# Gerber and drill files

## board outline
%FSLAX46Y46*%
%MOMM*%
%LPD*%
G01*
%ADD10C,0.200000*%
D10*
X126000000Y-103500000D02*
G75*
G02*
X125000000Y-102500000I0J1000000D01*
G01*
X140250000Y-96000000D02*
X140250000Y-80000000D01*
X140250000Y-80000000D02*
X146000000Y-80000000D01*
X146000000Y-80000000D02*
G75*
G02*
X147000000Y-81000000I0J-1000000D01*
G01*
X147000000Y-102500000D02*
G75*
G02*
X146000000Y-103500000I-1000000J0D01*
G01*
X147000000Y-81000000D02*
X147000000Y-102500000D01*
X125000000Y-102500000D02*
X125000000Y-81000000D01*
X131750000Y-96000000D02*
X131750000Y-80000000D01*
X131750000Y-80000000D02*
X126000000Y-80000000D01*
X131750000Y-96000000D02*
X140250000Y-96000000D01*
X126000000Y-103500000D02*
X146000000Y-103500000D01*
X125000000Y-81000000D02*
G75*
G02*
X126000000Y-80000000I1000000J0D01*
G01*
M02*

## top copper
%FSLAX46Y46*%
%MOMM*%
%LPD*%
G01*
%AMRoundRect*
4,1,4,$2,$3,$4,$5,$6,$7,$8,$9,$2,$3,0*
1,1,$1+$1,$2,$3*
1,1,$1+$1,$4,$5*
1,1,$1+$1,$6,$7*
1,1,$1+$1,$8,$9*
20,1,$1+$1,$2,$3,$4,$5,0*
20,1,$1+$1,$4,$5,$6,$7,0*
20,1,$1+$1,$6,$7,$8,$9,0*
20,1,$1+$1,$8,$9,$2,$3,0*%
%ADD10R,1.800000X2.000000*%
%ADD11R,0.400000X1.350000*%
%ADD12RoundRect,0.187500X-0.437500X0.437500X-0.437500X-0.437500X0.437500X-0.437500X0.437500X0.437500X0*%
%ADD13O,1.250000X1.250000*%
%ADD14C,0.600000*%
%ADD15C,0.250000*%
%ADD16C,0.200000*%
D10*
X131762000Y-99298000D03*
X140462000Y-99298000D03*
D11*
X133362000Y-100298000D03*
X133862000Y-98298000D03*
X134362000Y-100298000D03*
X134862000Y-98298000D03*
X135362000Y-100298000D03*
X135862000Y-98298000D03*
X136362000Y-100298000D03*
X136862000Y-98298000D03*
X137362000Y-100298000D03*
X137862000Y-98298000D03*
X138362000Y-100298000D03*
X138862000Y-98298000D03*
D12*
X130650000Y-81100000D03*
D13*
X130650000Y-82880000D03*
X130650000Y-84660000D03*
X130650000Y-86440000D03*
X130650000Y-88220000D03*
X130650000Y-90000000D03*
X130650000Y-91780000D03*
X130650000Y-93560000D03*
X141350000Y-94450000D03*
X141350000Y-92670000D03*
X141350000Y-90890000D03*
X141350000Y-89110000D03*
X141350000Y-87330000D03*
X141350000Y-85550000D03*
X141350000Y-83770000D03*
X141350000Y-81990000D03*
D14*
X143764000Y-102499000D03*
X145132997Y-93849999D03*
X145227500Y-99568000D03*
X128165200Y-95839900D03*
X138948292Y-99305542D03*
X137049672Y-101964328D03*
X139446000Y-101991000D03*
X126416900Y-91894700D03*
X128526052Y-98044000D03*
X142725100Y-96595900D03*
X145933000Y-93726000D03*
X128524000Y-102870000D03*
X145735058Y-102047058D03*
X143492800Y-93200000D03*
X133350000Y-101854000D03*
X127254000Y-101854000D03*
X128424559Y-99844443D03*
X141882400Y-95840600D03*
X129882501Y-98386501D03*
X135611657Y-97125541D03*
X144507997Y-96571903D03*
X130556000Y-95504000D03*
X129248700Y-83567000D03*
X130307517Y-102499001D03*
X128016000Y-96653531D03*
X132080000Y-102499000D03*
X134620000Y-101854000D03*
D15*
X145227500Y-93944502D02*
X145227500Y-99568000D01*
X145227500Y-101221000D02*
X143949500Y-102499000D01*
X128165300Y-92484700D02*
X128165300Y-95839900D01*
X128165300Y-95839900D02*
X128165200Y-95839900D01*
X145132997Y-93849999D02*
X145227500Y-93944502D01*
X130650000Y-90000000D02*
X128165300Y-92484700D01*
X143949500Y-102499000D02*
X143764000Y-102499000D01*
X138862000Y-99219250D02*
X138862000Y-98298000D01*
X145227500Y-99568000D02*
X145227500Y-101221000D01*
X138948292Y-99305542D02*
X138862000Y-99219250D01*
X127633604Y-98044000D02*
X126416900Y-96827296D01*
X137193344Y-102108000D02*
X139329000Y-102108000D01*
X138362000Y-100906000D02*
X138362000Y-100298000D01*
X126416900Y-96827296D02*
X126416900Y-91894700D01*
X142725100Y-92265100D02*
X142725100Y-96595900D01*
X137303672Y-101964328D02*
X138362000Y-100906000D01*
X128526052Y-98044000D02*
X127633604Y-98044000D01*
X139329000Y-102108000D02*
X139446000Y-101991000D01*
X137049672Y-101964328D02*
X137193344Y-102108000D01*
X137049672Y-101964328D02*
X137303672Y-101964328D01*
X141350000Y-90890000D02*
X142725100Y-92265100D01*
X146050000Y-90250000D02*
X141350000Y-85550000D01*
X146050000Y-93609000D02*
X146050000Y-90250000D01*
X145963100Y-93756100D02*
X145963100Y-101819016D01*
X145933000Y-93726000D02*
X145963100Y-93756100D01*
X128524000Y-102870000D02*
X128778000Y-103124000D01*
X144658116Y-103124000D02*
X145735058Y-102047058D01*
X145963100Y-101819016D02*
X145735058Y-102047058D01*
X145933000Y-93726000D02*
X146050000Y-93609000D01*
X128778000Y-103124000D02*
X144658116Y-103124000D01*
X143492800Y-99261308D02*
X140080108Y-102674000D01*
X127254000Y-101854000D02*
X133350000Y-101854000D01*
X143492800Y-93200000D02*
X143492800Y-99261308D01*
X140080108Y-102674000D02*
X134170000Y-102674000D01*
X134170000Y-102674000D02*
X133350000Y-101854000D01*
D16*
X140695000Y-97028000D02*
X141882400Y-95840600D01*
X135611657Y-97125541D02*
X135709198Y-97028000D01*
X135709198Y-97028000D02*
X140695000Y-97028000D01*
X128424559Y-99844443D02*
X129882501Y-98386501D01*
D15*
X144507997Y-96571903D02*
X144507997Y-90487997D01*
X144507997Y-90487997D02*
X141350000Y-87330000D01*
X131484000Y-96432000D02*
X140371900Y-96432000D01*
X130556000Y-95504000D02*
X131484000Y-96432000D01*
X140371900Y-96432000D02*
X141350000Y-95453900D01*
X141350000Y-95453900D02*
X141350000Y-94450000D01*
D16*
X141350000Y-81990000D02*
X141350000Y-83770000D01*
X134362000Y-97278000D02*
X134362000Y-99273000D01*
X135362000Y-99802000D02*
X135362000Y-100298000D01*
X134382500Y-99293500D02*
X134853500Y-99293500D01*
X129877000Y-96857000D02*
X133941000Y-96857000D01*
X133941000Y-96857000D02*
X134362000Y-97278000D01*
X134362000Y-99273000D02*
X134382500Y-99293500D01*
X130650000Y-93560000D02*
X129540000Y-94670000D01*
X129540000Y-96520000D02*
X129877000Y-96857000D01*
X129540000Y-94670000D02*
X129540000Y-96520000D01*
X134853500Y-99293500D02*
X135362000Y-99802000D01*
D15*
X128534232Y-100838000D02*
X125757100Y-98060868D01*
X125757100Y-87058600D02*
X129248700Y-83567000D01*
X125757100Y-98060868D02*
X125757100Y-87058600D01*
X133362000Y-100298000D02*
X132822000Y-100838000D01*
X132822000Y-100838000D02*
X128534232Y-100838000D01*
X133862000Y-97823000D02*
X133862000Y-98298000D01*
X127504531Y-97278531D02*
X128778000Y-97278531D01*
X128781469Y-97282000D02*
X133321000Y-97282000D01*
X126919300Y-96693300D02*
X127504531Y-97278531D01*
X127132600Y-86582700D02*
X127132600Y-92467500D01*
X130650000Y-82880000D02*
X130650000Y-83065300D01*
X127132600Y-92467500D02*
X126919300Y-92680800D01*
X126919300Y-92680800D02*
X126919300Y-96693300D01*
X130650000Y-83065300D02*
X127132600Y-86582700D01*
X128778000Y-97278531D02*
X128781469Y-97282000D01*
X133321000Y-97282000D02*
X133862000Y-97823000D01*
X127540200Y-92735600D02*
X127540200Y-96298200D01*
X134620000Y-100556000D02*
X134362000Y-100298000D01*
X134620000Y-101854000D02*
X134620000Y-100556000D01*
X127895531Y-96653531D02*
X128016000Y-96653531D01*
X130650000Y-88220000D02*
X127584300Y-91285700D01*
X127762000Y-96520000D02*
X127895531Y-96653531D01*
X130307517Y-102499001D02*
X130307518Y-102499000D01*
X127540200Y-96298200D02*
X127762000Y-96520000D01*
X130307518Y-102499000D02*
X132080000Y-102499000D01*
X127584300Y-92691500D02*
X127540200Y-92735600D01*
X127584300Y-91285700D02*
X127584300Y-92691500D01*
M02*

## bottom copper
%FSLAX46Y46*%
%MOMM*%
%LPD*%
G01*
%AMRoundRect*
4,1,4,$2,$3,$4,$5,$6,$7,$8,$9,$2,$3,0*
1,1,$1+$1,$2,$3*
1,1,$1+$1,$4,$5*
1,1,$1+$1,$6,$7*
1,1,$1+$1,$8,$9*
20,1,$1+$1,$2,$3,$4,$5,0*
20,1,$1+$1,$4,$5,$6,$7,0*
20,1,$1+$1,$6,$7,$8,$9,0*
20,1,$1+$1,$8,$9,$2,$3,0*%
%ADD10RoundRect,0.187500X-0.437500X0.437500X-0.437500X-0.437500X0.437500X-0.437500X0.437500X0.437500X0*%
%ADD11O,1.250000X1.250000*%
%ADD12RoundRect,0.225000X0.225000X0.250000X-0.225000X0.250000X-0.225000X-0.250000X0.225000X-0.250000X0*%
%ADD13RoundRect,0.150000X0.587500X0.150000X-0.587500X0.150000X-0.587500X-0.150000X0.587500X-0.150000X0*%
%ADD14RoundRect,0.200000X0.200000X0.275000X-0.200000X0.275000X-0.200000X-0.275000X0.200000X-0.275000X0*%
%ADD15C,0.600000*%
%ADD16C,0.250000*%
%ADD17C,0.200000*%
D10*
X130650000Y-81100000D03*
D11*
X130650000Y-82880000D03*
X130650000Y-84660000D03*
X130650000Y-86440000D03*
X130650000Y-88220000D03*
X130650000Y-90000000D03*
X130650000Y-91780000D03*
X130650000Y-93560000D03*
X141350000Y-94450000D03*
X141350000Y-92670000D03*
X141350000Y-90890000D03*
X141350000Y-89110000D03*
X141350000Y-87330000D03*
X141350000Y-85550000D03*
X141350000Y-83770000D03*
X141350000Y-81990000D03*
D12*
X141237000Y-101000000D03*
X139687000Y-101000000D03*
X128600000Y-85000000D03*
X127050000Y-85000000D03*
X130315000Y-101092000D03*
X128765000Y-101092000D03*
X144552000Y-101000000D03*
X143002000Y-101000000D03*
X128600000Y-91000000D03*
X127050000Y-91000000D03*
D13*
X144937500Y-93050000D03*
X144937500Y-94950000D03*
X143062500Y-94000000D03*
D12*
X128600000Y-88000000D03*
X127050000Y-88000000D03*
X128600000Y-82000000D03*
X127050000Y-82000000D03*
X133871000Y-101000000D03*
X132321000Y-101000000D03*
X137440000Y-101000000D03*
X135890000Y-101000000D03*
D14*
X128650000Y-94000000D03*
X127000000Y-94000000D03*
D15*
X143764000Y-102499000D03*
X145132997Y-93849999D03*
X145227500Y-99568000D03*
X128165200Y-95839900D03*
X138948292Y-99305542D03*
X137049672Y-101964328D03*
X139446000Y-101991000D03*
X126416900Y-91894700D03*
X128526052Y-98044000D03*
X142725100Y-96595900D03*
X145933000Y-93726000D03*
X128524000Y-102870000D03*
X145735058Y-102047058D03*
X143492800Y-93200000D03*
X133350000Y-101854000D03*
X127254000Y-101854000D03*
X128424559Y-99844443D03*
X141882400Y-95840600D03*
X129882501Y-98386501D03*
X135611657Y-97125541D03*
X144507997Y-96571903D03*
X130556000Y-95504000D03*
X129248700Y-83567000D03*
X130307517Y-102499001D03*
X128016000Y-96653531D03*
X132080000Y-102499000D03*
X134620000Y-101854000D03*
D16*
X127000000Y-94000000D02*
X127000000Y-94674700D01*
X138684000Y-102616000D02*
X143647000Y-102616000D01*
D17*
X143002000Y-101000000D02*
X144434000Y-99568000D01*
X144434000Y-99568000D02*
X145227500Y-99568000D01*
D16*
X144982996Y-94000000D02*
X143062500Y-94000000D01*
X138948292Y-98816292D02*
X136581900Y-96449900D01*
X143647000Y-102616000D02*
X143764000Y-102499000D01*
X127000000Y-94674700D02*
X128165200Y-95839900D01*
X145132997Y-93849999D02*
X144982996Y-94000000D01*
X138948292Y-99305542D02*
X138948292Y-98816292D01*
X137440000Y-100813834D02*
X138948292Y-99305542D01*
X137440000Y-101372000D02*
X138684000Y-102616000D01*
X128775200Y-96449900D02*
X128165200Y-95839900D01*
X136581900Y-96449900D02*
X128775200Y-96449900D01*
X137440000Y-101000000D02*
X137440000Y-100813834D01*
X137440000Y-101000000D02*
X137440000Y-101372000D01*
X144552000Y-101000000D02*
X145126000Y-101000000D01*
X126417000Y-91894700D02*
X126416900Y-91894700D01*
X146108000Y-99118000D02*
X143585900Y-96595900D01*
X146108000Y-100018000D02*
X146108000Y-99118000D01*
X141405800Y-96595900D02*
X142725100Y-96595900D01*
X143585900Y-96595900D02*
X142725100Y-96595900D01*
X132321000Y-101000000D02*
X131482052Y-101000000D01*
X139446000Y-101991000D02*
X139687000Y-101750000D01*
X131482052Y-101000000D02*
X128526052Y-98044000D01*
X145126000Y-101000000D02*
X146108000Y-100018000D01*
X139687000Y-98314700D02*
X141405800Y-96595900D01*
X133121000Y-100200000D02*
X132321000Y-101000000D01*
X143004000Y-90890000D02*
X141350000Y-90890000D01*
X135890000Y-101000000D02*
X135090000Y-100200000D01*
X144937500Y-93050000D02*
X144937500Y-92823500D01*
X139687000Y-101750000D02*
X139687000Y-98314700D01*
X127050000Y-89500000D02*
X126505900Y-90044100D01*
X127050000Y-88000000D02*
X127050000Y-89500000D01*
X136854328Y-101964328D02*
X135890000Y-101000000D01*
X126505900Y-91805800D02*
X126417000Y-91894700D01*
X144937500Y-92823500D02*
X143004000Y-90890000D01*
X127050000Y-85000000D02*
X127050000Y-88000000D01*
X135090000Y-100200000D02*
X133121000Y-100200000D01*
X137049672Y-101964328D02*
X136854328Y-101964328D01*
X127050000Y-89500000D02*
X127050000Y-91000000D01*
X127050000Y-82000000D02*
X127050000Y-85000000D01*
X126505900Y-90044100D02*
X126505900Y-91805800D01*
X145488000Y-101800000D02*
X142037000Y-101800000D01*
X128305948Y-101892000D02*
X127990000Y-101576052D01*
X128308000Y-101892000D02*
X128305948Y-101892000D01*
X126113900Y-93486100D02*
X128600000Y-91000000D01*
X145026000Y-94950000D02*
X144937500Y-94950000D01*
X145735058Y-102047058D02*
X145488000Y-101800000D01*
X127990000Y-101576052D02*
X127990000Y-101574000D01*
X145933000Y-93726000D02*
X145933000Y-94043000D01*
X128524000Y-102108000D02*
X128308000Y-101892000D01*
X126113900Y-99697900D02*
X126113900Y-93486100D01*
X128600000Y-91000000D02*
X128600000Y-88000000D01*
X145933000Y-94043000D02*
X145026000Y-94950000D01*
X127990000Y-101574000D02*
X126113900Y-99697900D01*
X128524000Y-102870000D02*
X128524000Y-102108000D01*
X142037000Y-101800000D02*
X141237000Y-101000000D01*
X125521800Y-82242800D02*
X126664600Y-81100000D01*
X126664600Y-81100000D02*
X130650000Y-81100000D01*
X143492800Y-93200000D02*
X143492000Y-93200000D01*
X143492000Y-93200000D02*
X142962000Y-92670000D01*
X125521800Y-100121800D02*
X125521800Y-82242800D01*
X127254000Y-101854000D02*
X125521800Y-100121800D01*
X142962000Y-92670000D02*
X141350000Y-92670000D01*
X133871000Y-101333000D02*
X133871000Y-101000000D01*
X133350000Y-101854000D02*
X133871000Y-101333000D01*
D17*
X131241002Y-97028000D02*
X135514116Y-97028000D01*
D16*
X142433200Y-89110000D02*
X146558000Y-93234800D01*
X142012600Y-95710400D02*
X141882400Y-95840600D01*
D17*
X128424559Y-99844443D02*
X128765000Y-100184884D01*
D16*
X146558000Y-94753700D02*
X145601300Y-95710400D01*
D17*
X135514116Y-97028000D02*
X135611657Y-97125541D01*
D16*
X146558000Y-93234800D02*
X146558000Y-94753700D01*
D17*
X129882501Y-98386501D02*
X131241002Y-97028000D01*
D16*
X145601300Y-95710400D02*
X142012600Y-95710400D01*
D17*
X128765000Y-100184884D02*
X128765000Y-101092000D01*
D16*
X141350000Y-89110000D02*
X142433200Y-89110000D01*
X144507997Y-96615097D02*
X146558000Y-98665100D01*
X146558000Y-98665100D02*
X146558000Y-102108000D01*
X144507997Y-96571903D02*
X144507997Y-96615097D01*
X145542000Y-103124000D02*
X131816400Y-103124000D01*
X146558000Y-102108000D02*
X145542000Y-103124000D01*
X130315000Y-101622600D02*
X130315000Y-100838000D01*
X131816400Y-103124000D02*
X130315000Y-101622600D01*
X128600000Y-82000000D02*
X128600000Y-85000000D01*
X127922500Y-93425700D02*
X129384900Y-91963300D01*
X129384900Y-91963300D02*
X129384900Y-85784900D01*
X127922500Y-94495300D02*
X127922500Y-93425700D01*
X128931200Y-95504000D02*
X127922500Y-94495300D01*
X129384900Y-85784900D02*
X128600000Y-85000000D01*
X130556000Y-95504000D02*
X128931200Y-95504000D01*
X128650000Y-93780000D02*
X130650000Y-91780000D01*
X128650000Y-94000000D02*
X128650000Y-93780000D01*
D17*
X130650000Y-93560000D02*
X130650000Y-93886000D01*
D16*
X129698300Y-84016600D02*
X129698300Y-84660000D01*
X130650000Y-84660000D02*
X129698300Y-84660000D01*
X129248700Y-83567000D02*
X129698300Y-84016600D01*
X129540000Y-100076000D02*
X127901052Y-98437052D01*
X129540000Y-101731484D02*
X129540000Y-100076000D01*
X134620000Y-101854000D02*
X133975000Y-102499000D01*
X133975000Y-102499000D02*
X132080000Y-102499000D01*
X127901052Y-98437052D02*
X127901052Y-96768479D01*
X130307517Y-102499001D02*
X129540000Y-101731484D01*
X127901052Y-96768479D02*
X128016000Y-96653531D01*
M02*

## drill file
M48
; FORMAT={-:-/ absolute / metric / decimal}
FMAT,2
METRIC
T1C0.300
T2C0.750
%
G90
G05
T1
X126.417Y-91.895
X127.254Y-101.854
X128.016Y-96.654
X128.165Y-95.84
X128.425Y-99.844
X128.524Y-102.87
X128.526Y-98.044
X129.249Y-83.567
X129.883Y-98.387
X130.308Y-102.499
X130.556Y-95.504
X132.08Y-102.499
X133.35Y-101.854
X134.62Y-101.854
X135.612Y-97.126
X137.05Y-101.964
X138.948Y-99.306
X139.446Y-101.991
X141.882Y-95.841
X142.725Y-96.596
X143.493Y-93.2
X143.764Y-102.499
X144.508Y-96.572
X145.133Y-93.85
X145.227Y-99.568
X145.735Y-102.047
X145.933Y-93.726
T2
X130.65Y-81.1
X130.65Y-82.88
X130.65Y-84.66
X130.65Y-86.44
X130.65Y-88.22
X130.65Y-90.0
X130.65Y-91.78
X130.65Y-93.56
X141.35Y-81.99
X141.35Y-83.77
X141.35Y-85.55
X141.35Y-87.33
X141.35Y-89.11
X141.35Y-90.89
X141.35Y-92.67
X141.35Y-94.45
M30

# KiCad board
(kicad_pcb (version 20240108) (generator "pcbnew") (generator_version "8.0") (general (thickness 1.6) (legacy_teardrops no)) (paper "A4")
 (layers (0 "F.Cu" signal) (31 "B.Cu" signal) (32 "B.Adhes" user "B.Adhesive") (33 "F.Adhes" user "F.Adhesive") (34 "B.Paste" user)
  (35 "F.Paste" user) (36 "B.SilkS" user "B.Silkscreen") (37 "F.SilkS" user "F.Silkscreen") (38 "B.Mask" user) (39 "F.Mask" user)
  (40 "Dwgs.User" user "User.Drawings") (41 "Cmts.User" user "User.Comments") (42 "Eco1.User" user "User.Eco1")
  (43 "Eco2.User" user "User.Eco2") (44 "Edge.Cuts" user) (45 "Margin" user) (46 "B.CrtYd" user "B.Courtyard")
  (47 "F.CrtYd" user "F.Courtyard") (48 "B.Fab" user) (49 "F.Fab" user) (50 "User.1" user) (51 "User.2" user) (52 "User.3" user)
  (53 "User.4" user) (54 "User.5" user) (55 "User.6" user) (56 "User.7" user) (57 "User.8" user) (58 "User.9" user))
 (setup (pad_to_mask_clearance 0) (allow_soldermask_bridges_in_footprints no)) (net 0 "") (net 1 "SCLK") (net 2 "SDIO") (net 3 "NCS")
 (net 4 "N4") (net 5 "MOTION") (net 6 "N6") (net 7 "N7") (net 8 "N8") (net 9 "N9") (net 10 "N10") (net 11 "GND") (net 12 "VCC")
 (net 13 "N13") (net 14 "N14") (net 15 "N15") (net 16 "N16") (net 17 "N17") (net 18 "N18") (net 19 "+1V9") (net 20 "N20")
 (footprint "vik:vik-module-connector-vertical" (layer "F.Cu") (at 136.112 99.298)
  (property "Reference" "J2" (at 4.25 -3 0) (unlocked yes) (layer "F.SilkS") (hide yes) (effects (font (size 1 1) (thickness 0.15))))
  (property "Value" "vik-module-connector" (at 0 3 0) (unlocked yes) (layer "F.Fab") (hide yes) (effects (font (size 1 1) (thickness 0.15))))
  (pad "" smd rect (at -4.35 0) (size 1.8 2) (layers "F.Cu" "F.Paste" "F.Mask") (thermal_bridge_angle 45))
  (pad "" smd rect (at 4.35 0) (size 1.8 2) (layers "F.Cu" "F.Paste" "F.Mask") (thermal_bridge_angle 45))
  (pad "1" smd rect (at -2.75 1) (size 0.4 1.35) (layers "F.Cu" "F.Paste" "F.Mask") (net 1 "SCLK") (thermal_bridge_angle 45))
  (pad "2" smd rect (at -2.25 -1) (size 0.4 1.35) (layers "F.Cu" "F.Paste" "F.Mask") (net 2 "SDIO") (thermal_bridge_angle 45))
  (pad "3" smd rect (at -1.75 1) (size 0.4 1.35) (layers "F.Cu" "F.Paste" "F.Mask") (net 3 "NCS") (thermal_bridge_angle 45))
  (pad "4" smd rect (at -1.25 -1) (size 0.4 1.35) (layers "F.Cu" "F.Paste" "F.Mask") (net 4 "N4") (thermal_bridge_angle 45))
  (pad "5" smd rect (at -0.75 1) (size 0.4 1.35) (layers "F.Cu" "F.Paste" "F.Mask") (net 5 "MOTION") (thermal_bridge_angle 45))
  (pad "6" smd rect (at -0.25 -1) (size 0.4 1.35) (layers "F.Cu" "F.Paste" "F.Mask") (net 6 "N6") (thermal_bridge_angle 45))
  (pad "7" smd rect (at 0.25 1) (size 0.4 1.35) (layers "F.Cu" "F.Paste" "F.Mask") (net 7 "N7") (thermal_bridge_angle 45))
  (pad "8" smd rect (at 0.75 -1) (size 0.4 1.35) (layers "F.Cu" "F.Paste" "F.Mask") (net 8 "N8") (thermal_bridge_angle 45))
  (pad "9" smd rect (at 1.25 1) (size 0.4 1.35) (layers "F.Cu" "F.Paste" "F.Mask") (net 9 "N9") (thermal_bridge_angle 45))
  (pad "10" smd rect (at 1.75 -1) (size 0.4 1.35) (layers "F.Cu" "F.Paste" "F.Mask") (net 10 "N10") (thermal_bridge_angle 45))
  (pad "11" smd rect (at 2.25 1) (size 0.4 1.35) (layers "F.Cu" "F.Paste" "F.Mask") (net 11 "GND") (thermal_bridge_angle 45))
  (pad "12" smd rect (at 2.75 -1) (size 0.4 1.35) (layers "F.Cu" "F.Paste" "F.Mask") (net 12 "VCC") (thermal_bridge_angle 45)))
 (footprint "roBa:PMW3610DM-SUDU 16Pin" (layer "F.Cu") (at 136 87.268 90)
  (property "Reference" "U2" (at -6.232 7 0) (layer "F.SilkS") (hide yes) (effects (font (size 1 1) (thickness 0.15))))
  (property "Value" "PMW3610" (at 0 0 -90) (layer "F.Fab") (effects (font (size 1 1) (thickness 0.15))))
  (pad "1" thru_hole roundrect (at 6.168 -5.35 270) (size 1.25 1.25) (drill 0.75) (layers "*.Cu" "*.Mask") (remove_unused_layers no)
   (roundrect_rratio 0.15) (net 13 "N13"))
  (pad "2" thru_hole oval (at 4.388 -5.35 270) (size 1.25 1.25) (drill 0.75) (layers "*.Cu" "*.Mask") (remove_unused_layers no)
   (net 2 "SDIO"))
  (pad "3" thru_hole oval (at 2.608 -5.35 270) (size 1.25 1.25) (drill 0.75) (layers "*.Cu" "*.Mask") (remove_unused_layers no)
   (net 1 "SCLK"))
  (pad "4" thru_hole oval (at 0.828 -5.35 270) (size 1.25 1.25) (drill 0.75) (layers "*.Cu" "*.Mask") (remove_unused_layers no)
   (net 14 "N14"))
  (pad "5" thru_hole oval (at -0.952 -5.35 270) (size 1.25 1.25) (drill 0.75) (layers "*.Cu" "*.Mask") (remove_unused_layers no)
   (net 3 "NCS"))
  (pad "6" thru_hole oval (at -2.732 -5.35 270) (size 1.25 1.25) (drill 0.75) (layers "*.Cu" "*.Mask") (remove_unused_layers no)
   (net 12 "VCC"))
  (pad "7" thru_hole oval (at -4.512 -5.35 270) (size 1.25 1.25) (drill 0.75) (layers "*.Cu" "*.Mask") (remove_unused_layers no)
   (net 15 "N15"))
  (pad "8" thru_hole oval (at -6.292 -5.35 270) (size 1.25 1.25) (drill 0.75) (layers "*.Cu" "*.Mask") (remove_unused_layers no)
   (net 5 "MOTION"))
  (pad "9" thru_hole oval (at -7.182 5.35 270) (size 1.25 1.25) (drill 0.75) (layers "*.Cu" "*.Mask") (remove_unused_layers no)
   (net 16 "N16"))
  (pad "10" thru_hole oval (at -5.402 5.35 270) (size 1.25 1.25) (drill 0.75) (layers "*.Cu" "*.Mask") (remove_unused_layers no)
   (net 13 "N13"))
  (pad "11" thru_hole oval (at -3.622 5.35 270) (size 1.25 1.25) (drill 0.75) (layers "*.Cu" "*.Mask") (remove_unused_layers no)
   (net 11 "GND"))
  (pad "12" thru_hole oval (at -1.842 5.35 270) (size 1.25 1.25) (drill 0.75) (layers "*.Cu" "*.Mask") (remove_unused_layers no)
   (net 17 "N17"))
  (pad "13" thru_hole oval (at -0.062 5.35 270) (size 1.25 1.25) (drill 0.75) (layers "*.Cu" "*.Mask") (remove_unused_layers no)
   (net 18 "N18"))
  (pad "14" thru_hole oval (at 1.718 5.35 270) (size 1.25 1.25) (drill 0.75) (layers "*.Cu" "*.Mask") (remove_unused_layers no)
   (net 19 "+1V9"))
  (pad "15" thru_hole oval (at 3.498 5.35 270) (size 1.25 1.25) (drill 0.75) (layers "*.Cu" "*.Mask") (remove_unused_layers no)
   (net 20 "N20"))
  (pad "16" thru_hole oval (at 5.278 5.35 270) (size 1.25 1.25) (drill 0.75) (layers "*.Cu" "*.Mask") (remove_unused_layers no)
   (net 20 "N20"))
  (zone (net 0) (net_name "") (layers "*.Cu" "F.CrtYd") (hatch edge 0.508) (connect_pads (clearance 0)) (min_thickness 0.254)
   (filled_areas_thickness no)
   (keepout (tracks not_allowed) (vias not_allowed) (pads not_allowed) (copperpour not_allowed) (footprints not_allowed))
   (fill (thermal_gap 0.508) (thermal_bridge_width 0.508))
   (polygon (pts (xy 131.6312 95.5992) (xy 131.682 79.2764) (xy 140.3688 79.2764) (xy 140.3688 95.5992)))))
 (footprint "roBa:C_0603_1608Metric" (layer "B.Cu") (at 140.462 101 180)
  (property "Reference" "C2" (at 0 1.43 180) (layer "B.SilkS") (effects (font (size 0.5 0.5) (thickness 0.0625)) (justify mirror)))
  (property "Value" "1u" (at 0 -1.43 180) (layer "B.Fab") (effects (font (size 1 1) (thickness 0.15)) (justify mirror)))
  (pad "1" smd roundrect (at -0.775 0 180) (size 0.9 0.95) (layers "B.Cu" "B.Paste" "B.Mask") (roundrect_rratio 0.25) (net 19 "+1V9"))
  (pad "2" smd roundrect (at 0.775 0 180) (size 0.9 0.95) (layers "B.Cu" "B.Paste" "B.Mask") (roundrect_rratio 0.25) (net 11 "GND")))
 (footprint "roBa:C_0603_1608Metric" (layer "B.Cu") (at 127.825 85 180)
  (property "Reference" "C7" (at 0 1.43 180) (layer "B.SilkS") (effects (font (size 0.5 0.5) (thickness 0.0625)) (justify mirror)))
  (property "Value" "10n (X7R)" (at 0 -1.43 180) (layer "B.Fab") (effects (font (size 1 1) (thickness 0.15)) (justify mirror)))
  (pad "1" smd roundrect (at -0.775 0 180) (size 0.9 0.95) (layers "B.Cu" "B.Paste" "B.Mask") (roundrect_rratio 0.25) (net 16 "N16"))
  (pad "2" smd roundrect (at 0.775 0 180) (size 0.9 0.95) (layers "B.Cu" "B.Paste" "B.Mask") (roundrect_rratio 0.25) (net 11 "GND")))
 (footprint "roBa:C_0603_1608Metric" (layer "B.Cu") (at 129.54 101.092 180)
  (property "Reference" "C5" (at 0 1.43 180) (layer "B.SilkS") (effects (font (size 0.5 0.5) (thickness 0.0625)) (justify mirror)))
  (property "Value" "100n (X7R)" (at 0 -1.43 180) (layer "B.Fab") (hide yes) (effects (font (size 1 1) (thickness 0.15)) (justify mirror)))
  (pad "1" smd roundrect (at -0.775 0 180) (size 0.9 0.95) (layers "B.Cu" "B.Paste" "B.Mask") (roundrect_rratio 0.25) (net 18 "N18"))
  (pad "2" smd roundrect (at 0.775 0 180) (size 0.9 0.95) (layers "B.Cu" "B.Paste" "B.Mask") (roundrect_rratio 0.25) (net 17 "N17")))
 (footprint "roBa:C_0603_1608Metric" (layer "B.Cu") (at 143.777 101 180)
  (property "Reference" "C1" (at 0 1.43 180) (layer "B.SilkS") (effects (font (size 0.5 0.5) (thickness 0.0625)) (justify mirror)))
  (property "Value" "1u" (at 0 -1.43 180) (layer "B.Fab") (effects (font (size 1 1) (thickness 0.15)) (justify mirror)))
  (pad "1" smd roundrect (at -0.775 0 180) (size 0.9 0.95) (layers "B.Cu" "B.Paste" "B.Mask") (roundrect_rratio 0.25) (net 11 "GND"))
  (pad "2" smd roundrect (at 0.775 0 180) (size 0.9 0.95) (layers "B.Cu" "B.Paste" "B.Mask") (roundrect_rratio 0.25) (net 12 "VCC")))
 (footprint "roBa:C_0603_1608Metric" (layer "B.Cu") (at 127.825 91 180)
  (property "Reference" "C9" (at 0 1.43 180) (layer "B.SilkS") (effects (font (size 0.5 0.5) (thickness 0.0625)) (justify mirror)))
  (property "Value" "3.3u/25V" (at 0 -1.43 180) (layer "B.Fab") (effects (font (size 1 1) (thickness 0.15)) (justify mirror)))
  (pad "1" smd roundrect (at -0.775 0 180) (size 0.9 0.95) (layers "B.Cu" "B.Paste" "B.Mask") (roundrect_rratio 0.25) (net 19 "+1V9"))
  (pad "2" smd roundrect (at 0.775 0 180) (size 0.9 0.95) (layers "B.Cu" "B.Paste" "B.Mask") (roundrect_rratio 0.25) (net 11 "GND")))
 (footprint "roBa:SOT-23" (layer "B.Cu") (at 144 94 180)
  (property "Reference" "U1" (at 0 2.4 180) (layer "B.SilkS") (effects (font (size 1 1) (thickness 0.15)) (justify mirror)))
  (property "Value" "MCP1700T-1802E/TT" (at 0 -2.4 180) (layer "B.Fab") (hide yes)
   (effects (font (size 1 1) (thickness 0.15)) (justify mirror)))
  (pad "1" smd roundrect (at -0.9375 0.95 180) (size 1.475 0.6) (layers "B.Cu" "B.Paste" "B.Mask") (roundrect_rratio 0.25) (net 11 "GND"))
  (pad "2" smd roundrect (at -0.9375 -0.95 180) (size 1.475 0.6) (layers "B.Cu" "B.Paste" "B.Mask") (roundrect_rratio 0.25) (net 19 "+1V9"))
  (pad "3" smd roundrect (at 0.9375 0 180) (size 1.475 0.6) (layers "B.Cu" "B.Paste" "B.Mask") (roundrect_rratio 0.25) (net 12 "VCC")))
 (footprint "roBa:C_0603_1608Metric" (layer "B.Cu") (at 127.825 88 180)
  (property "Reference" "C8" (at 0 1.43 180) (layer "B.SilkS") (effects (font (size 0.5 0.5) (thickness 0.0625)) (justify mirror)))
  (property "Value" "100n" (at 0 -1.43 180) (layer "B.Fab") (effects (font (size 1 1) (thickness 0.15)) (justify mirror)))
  (pad "1" smd roundrect (at -0.775 0 180) (size 0.9 0.95) (layers "B.Cu" "B.Paste" "B.Mask") (roundrect_rratio 0.25) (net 19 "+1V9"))
  (pad "2" smd roundrect (at 0.775 0 180) (size 0.9 0.95) (layers "B.Cu" "B.Paste" "B.Mask") (roundrect_rratio 0.25) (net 11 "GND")))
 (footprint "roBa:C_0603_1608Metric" (layer "B.Cu") (at 127.825 82 180)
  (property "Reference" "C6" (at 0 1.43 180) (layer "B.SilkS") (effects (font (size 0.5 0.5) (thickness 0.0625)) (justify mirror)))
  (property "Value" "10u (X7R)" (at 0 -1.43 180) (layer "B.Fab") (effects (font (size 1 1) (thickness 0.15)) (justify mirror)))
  (pad "1" smd roundrect (at -0.775 0 180) (size 0.9 0.95) (layers "B.Cu" "B.Paste" "B.Mask") (roundrect_rratio 0.25) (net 16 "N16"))
  (pad "2" smd roundrect (at 0.775 0 180) (size 0.9 0.95) (layers "B.Cu" "B.Paste" "B.Mask") (roundrect_rratio 0.25) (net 11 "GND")))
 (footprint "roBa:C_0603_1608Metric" (layer "B.Cu") (at 133.096 101 180)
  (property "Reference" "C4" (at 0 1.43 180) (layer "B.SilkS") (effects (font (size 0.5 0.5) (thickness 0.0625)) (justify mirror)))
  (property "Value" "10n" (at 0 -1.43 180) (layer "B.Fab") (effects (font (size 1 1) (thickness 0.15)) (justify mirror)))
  (pad "1" smd roundrect (at -0.775 0 180) (size 0.9 0.95) (layers "B.Cu" "B.Paste" "B.Mask") (roundrect_rratio 0.25) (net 13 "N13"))
  (pad "2" smd roundrect (at 0.775 0 180) (size 0.9 0.95) (layers "B.Cu" "B.Paste" "B.Mask") (roundrect_rratio 0.25) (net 11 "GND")))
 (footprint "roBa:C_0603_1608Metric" (layer "B.Cu") (at 136.665 101 180)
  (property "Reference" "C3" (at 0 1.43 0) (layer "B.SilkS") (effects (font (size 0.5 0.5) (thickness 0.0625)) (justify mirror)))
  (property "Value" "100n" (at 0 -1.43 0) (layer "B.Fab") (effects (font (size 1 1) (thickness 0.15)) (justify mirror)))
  (pad "1" smd roundrect (at -0.775 0 180) (size 0.9 0.95) (layers "B.Cu" "B.Paste" "B.Mask") (roundrect_rratio 0.25) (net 12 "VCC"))
  (pad "2" smd roundrect (at 0.775 0 180) (size 0.9 0.95) (layers "B.Cu" "B.Paste" "B.Mask") (roundrect_rratio 0.25) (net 11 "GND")))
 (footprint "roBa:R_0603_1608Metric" (layer "B.Cu") (at 127.825 94 180)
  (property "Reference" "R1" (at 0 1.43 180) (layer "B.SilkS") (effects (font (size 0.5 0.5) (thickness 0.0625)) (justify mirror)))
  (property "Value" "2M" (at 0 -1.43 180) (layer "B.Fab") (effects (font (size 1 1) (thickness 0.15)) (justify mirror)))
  (pad "1" smd roundrect (at -0.825 0 180) (size 0.8 0.95) (layers "B.Cu" "B.Paste" "B.Mask") (roundrect_rratio 0.25) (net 15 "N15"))
  (pad "2" smd roundrect (at 0.825 0 180) (size 0.8 0.95) (layers "B.Cu" "B.Paste" "B.Mask") (roundrect_rratio 0.25) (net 12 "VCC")))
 (gr_arc (start 126 103.5) (mid 125.292893 103.207107) (end 125 102.5) (stroke (width 0.2) (type default)) (layer "Edge.Cuts"))
 (gr_line (start 140.25 96) (end 140.25 80) (stroke (width 0.2) (type default)) (layer "Edge.Cuts"))
 (gr_line (start 140.25 80) (end 146 80) (stroke (width 0.2) (type default)) (layer "Edge.Cuts"))
 (gr_arc (start 146 80) (mid 146.707107 80.292893) (end 147 81) (stroke (width 0.2) (type default)) (layer "Edge.Cuts"))
 (gr_arc (start 147 102.5) (mid 146.707107 103.207107) (end 146 103.5) (stroke (width 0.2) (type default)) (layer "Edge.Cuts"))
 (gr_line (start 147 81) (end 147 102.5) (stroke (width 0.2) (type default)) (layer "Edge.Cuts"))
 (gr_line (start 125 102.5) (end 125 81) (stroke (width 0.2) (type default)) (layer "Edge.Cuts"))
 (gr_line (start 131.75 96) (end 131.75 80) (stroke (width 0.2) (type default)) (layer "Edge.Cuts"))
 (gr_line (start 131.75 80) (end 126 80) (stroke (width 0.2) (type default)) (layer "Edge.Cuts"))
 (gr_line (start 131.75 96) (end 140.25 96) (stroke (width 0.2) (type default)) (layer "Edge.Cuts"))
 (gr_line (start 126 103.5) (end 146 103.5) (stroke (width 0.2) (type default)) (layer "Edge.Cuts"))
 (gr_arc (start 125 81) (mid 125.292893 80.292893) (end 126 80) (stroke (width 0.2) (type default)) (layer "Edge.Cuts"))
 (segment (start 145.2275 93.944502) (end 145.2275 99.568) (width 0.25) (layer "F.Cu") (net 12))
 (segment (start 145.2275 101.221) (end 143.9495 102.499) (width 0.25) (layer "F.Cu") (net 12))
 (segment (start 128.1653 92.4847) (end 128.1653 95.8399) (width 0.25) (layer "F.Cu") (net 12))
 (segment (start 128.1653 95.8399) (end 128.1652 95.8399) (width 0.25) (layer "F.Cu") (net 12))
 (segment (start 145.132997 93.849999) (end 145.2275 93.944502) (width 0.25) (layer "F.Cu") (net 12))
 (segment (start 130.65 90) (end 128.1653 92.4847) (width 0.25) (layer "F.Cu") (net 12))
 (segment (start 143.9495 102.499) (end 143.764 102.499) (width 0.25) (layer "F.Cu") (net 12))
 (segment (start 138.862 99.21925) (end 138.862 98.298) (width 0.25) (layer "F.Cu") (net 12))
 (segment (start 145.2275 99.568) (end 145.2275 101.221) (width 0.25) (layer "F.Cu") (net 12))
 (segment (start 138.948292 99.305542) (end 138.862 99.21925) (width 0.25) (layer "F.Cu") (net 12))
 (via (at 143.764 102.499) (size 0.6) (drill 0.3) (layers "F.Cu" "B.Cu") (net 12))
 (via (at 145.132997 93.849999) (size 0.6) (drill 0.3) (layers "F.Cu" "B.Cu") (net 12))
 (via (at 145.2275 99.568) (size 0.6) (drill 0.3) (layers "F.Cu" "B.Cu") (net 12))
 (via (at 128.1652 95.8399) (size 0.6) (drill 0.3) (layers "F.Cu" "B.Cu") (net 12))
 (via (at 138.948292 99.305542) (size 0.6) (drill 0.3) (layers "F.Cu" "B.Cu") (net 12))
 (segment (start 127 94) (end 127 94.6747) (width 0.25) (layer "B.Cu") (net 12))
 (segment (start 138.684 102.616) (end 143.647 102.616) (width 0.25) (layer "B.Cu") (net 12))
 (segment (start 143.002 101) (end 144.434 99.568) (width 0.2) (layer "B.Cu") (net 12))
 (segment (start 144.434 99.568) (end 145.2275 99.568) (width 0.2) (layer "B.Cu") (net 12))
 (segment (start 144.982996 94) (end 143.0625 94) (width 0.25) (layer "B.Cu") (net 12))
 (segment (start 138.948292 98.816292) (end 136.5819 96.4499) (width 0.25) (layer "B.Cu") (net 12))
 (segment (start 143.647 102.616) (end 143.764 102.499) (width 0.25) (layer "B.Cu") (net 12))
 (segment (start 127 94.6747) (end 128.1652 95.8399) (width 0.25) (layer "B.Cu") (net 12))
 (segment (start 145.132997 93.849999) (end 144.982996 94) (width 0.25) (layer "B.Cu") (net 12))
 (segment (start 138.948292 99.305542) (end 138.948292 98.816292) (width 0.25) (layer "B.Cu") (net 12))
 (segment (start 137.44 100.813834) (end 138.948292 99.305542) (width 0.25) (layer "B.Cu") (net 12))
 (segment (start 137.44 101.372) (end 138.684 102.616) (width 0.25) (layer "B.Cu") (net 12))
 (segment (start 128.7752 96.4499) (end 128.1652 95.8399) (width 0.25) (layer "B.Cu") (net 12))
 (segment (start 136.5819 96.4499) (end 128.7752 96.4499) (width 0.25) (layer "B.Cu") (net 12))
 (segment (start 137.44 101) (end 137.44 100.813834) (width 0.25) (layer "B.Cu") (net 12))
 (segment (start 137.44 101) (end 137.44 101.372) (width 0.25) (layer "B.Cu") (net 12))
 (segment (start 127.633604 98.044) (end 126.4169 96.827296) (width 0.25) (layer "F.Cu") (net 11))
 (segment (start 137.193344 102.108) (end 139.329 102.108) (width 0.25) (layer "F.Cu") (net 11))
 (segment (start 138.362 100.906) (end 138.362 100.298) (width 0.25) (layer "F.Cu") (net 11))
 (segment (start 126.4169 96.827296) (end 126.4169 91.8947) (width 0.25) (layer "F.Cu") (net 11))
 (segment (start 142.7251 92.2651) (end 142.7251 96.5959) (width 0.25) (layer "F.Cu") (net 11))
 (segment (start 137.303672 101.964328) (end 138.362 100.906) (width 0.25) (layer "F.Cu") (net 11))
 (segment (start 128.526052 98.044) (end 127.633604 98.044) (width 0.25) (layer "F.Cu") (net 11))
 (segment (start 139.329 102.108) (end 139.446 101.991) (width 0.25) (layer "F.Cu") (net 11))
 (segment (start 137.049672 101.964328) (end 137.193344 102.108) (width 0.25) (layer "F.Cu") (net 11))
 (segment (start 137.049672 101.964328) (end 137.303672 101.964328) (width 0.25) (layer "F.Cu") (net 11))
 (segment (start 141.35 90.89) (end 142.7251 92.2651) (width 0.25) (layer "F.Cu") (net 11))
 (via (at 137.049672 101.964328) (size 0.6) (drill 0.3) (layers "F.Cu" "B.Cu") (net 11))
 (via (at 139.446 101.991) (size 0.6) (drill 0.3) (layers "F.Cu" "B.Cu") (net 11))
 (via (at 126.4169 91.8947) (size 0.6) (drill 0.3) (layers "F.Cu" "B.Cu") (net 11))
 (via (at 128.526052 98.044) (size 0.6) (drill 0.3) (layers "F.Cu" "B.Cu") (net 11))
 (via (at 142.7251 96.5959) (size 0.6) (drill 0.3) (layers "F.Cu" "B.Cu") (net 11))
 (segment (start 144.552 101) (end 145.126 101) (width 0.25) (layer "B.Cu") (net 11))
 (segment (start 126.417 91.8947) (end 126.4169 91.8947) (width 0.25) (layer "B.Cu") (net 11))
 (segment (start 146.108 99.118) (end 143.5859 96.5959) (width 0.25) (layer "B.Cu") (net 11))
 (segment (start 146.108 100.018) (end 146.108 99.118) (width 0.25) (layer "B.Cu") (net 11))
 (segment (start 141.4058 96.5959) (end 142.7251 96.5959) (width 0.25) (layer "B.Cu") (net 11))
 (segment (start 143.5859 96.5959) (end 142.7251 96.5959) (width 0.25) (layer "B.Cu") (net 11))
 (segment (start 132.321 101) (end 131.482052 101) (width 0.25) (layer "B.Cu") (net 11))
 (segment (start 139.446 101.991) (end 139.687 101.75) (width 0.25) (layer "B.Cu") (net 11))
 (segment (start 131.482052 101) (end 128.526052 98.044) (width 0.25) (layer "B.Cu") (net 11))
 (segment (start 145.126 101) (end 146.108 100.018) (width 0.25) (layer "B.Cu") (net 11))
 (segment (start 139.687 98.3147) (end 141.4058 96.5959) (width 0.25) (layer "B.Cu") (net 11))
 (segment (start 133.121 100.2) (end 132.321 101) (width 0.25) (layer "B.Cu") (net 11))
 (segment (start 143.004 90.89) (end 141.35 90.89) (width 0.25) (layer "B.Cu") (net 11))
 (segment (start 135.89 101) (end 135.09 100.2) (width 0.25) (layer "B.Cu") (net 11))
 (segment (start 144.9375 93.05) (end 144.9375 92.8235) (width 0.25) (layer "B.Cu") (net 11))
 (segment (start 139.687 101.75) (end 139.687 98.3147) (width 0.25) (layer "B.Cu") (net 11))
 (segment (start 127.05 89.5) (end 126.5059 90.0441) (width 0.25) (layer "B.Cu") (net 11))
 (segment (start 127.05 88) (end 127.05 89.5) (width 0.25) (layer "B.Cu") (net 11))
 (segment (start 136.854328 101.964328) (end 135.89 101) (width 0.25) (layer "B.Cu") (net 11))
 (segment (start 126.5059 91.8058) (end 126.417 91.8947) (width 0.25) (layer "B.Cu") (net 11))
 (segment (start 144.9375 92.8235) (end 143.004 90.89) (width 0.25) (layer "B.Cu") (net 11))
 (segment (start 127.05 85) (end 127.05 88) (width 0.25) (layer "B.Cu") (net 11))
 (segment (start 135.09 100.2) (end 133.121 100.2) (width 0.25) (layer "B.Cu") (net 11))
 (segment (start 137.049672 101.964328) (end 136.854328 101.964328) (width 0.25) (layer "B.Cu") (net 11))
 (segment (start 127.05 89.5) (end 127.05 91) (width 0.25) (layer "B.Cu") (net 11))
 (segment (start 127.05 82) (end 127.05 85) (width 0.25) (layer "B.Cu") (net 11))
 (segment (start 126.5059 90.0441) (end 126.5059 91.8058) (width 0.25) (layer "B.Cu") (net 11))
 (segment (start 146.05 90.25) (end 141.35 85.55) (width 0.25) (layer "F.Cu") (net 19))
 (segment (start 146.05 93.609) (end 146.05 90.25) (width 0.25) (layer "F.Cu") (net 19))
 (segment (start 145.9631 93.7561) (end 145.9631 101.819016) (width 0.25) (layer "F.Cu") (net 19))
 (segment (start 145.933 93.726) (end 145.9631 93.7561) (width 0.25) (layer "F.Cu") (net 19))
 (segment (start 128.524 102.87) (end 128.778 103.124) (width 0.25) (layer "F.Cu") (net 19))
 (segment (start 144.658116 103.124) (end 145.735058 102.047058) (width 0.25) (layer "F.Cu") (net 19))
 (segment (start 145.9631 101.819016) (end 145.735058 102.047058) (width 0.25) (layer "F.Cu") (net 19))
 (segment (start 145.933 93.726) (end 146.05 93.609) (width 0.25) (layer "F.Cu") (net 19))
 (segment (start 128.778 103.124) (end 144.658116 103.124) (width 0.25) (layer "F.Cu") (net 19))
 (via (at 145.933 93.726) (size 0.6) (drill 0.3) (layers "F.Cu" "B.Cu") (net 19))
 (via (at 128.524 102.87) (size 0.6) (drill 0.3) (layers "F.Cu" "B.Cu") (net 19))
 (via (at 145.735058 102.047058) (size 0.6) (drill 0.3) (layers "F.Cu" "B.Cu") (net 19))
 (segment (start 145.488 101.8) (end 142.037 101.8) (width 0.25) (layer "B.Cu") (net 19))
 (segment (start 128.305948 101.892) (end 127.99 101.576052) (width 0.25) (layer "B.Cu") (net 19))
 (segment (start 128.308 101.892) (end 128.305948 101.892) (width 0.25) (layer "B.Cu") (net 19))
 (segment (start 126.1139 93.4861) (end 128.6 91) (width 0.25) (layer "B.Cu") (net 19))
 (segment (start 145.026 94.95) (end 144.9375 94.95) (width 0.25) (layer "B.Cu") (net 19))
 (segment (start 145.735058 102.047058) (end 145.488 101.8) (width 0.25) (layer "B.Cu") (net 19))
 (segment (start 127.99 101.576052) (end 127.99 101.574) (width 0.25) (layer "B.Cu") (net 19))
 (segment (start 145.933 93.726) (end 145.933 94.043) (width 0.25) (layer "B.Cu") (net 19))
 (segment (start 128.524 102.108) (end 128.308 101.892) (width 0.25) (layer "B.Cu") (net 19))
 (segment (start 126.1139 99.6979) (end 126.1139 93.4861) (width 0.25) (layer "B.Cu") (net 19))
 (segment (start 128.6 91) (end 128.6 88) (width 0.25) (layer "B.Cu") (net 19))
 (segment (start 145.933 94.043) (end 145.026 94.95) (width 0.25) (layer "B.Cu") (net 19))
 (segment (start 127.99 101.574) (end 126.1139 99.6979) (width 0.25) (layer "B.Cu") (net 19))
 (segment (start 128.524 102.87) (end 128.524 102.108) (width 0.25) (layer "B.Cu") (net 19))
 (segment (start 142.037 101.8) (end 141.237 101) (width 0.25) (layer "B.Cu") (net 19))
 (segment (start 143.4928 99.261308) (end 140.080108 102.674) (width 0.25) (layer "F.Cu") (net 13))
 (segment (start 127.254 101.854) (end 133.35 101.854) (width 0.25) (layer "F.Cu") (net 13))
 (segment (start 143.4928 93.2) (end 143.4928 99.261308) (width 0.25) (layer "F.Cu") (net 13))
 (segment (start 140.080108 102.674) (end 134.17 102.674) (width 0.25) (layer "F.Cu") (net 13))
 (segment (start 134.17 102.674) (end 133.35 101.854) (width 0.25) (layer "F.Cu") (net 13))
 (via (at 143.4928 93.2) (size 0.6) (drill 0.3) (layers "F.Cu" "B.Cu") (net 13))
 (via (at 133.35 101.854) (size 0.6) (drill 0.3) (layers "F.Cu" "B.Cu") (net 13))
 (via (at 127.254 101.854) (size 0.6) (drill 0.3) (layers "F.Cu" "B.Cu") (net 13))
 (segment (start 125.5218 82.2428) (end 126.6646 81.1) (width 0.25) (layer "B.Cu") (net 13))
 (segment (start 126.6646 81.1) (end 130.65 81.1) (width 0.25) (layer "B.Cu") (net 13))
 (segment (start 143.4928 93.2) (end 143.492 93.2) (width 0.25) (layer "B.Cu") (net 13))
 (segment (start 143.492 93.2) (end 142.962 92.67) (width 0.25) (layer "B.Cu") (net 13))
 (segment (start 125.5218 100.1218) (end 125.5218 82.2428) (width 0.25) (layer "B.Cu") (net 13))
 (segment (start 127.254 101.854) (end 125.5218 100.1218) (width 0.25) (layer "B.Cu") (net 13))
 (segment (start 142.962 92.67) (end 141.35 92.67) (width 0.25) (layer "B.Cu") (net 13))
 (segment (start 133.871 101.333) (end 133.871 101) (width 0.25) (layer "B.Cu") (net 13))
 (segment (start 133.35 101.854) (end 133.871 101.333) (width 0.25) (layer "B.Cu") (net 13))
 (segment (start 140.695 97.028) (end 141.8824 95.8406) (width 0.2) (layer "F.Cu") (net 17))
 (segment (start 135.611657 97.125541) (end 135.709198 97.028) (width 0.2) (layer "F.Cu") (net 17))
 (segment (start 135.709198 97.028) (end 140.695 97.028) (width 0.2) (layer "F.Cu") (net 17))
 (segment (start 128.424559 99.844443) (end 129.882501 98.386501) (width 0.2) (layer "F.Cu") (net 17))
 (via (at 128.424559 99.844443) (size 0.6) (drill 0.3) (layers "F.Cu" "B.Cu") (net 17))
 (via (at 141.8824 95.8406) (size 0.6) (drill 0.3) (layers "F.Cu" "B.Cu") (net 17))
 (via (at 129.882501 98.386501) (size 0.6) (drill 0.3) (layers "F.Cu" "B.Cu") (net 17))
 (via (at 135.611657 97.125541) (size 0.6) (drill 0.3) (layers "F.Cu" "B.Cu") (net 17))
 (segment (start 131.241002 97.028) (end 135.514116 97.028) (width 0.2) (layer "B.Cu") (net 17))
 (segment (start 142.4332 89.11) (end 146.558 93.2348) (width 0.25) (layer "B.Cu") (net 17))
 (segment (start 142.0126 95.7104) (end 141.8824 95.8406) (width 0.25) (layer "B.Cu") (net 17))
 (segment (start 128.424559 99.844443) (end 128.765 100.184884) (width 0.2) (layer "B.Cu") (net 17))
 (segment (start 146.558 94.7537) (end 145.6013 95.7104) (width 0.25) (layer "B.Cu") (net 17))
 (segment (start 135.514116 97.028) (end 135.611657 97.125541) (width 0.2) (layer "B.Cu") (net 17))
 (segment (start 146.558 93.2348) (end 146.558 94.7537) (width 0.25) (layer "B.Cu") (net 17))
 (segment (start 129.882501 98.386501) (end 131.241002 97.028) (width 0.2) (layer "B.Cu") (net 17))
 (segment (start 145.6013 95.7104) (end 142.0126 95.7104) (width 0.25) (layer "B.Cu") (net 17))
 (segment (start 128.765 100.184884) (end 128.765 101.092) (width 0.2) (layer "B.Cu") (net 17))
 (segment (start 141.35 89.11) (end 142.4332 89.11) (width 0.25) (layer "B.Cu") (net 17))
 (segment (start 144.507997 96.571903) (end 144.507997 90.487997) (width 0.25) (layer "F.Cu") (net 18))
 (segment (start 144.507997 90.487997) (end 141.35 87.33) (width 0.25) (layer "F.Cu") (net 18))
 (via (at 144.507997 96.571903) (size 0.6) (drill 0.3) (layers "F.Cu" "B.Cu") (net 18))
 (segment (start 144.507997 96.615097) (end 146.558 98.6651) (width 0.25) (layer "B.Cu") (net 18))
 (segment (start 146.558 98.6651) (end 146.558 102.108) (width 0.25) (layer "B.Cu") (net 18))
 (segment (start 144.507997 96.571903) (end 144.507997 96.615097) (width 0.25) (layer "B.Cu") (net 18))
 (segment (start 145.542 103.124) (end 131.8164 103.124) (width 0.25) (layer "B.Cu") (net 18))
 (segment (start 146.558 102.108) (end 145.542 103.124) (width 0.25) (layer "B.Cu") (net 18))
 (segment (start 130.315 101.6226) (end 130.315 100.838) (width 0.25) (layer "B.Cu") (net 18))
 (segment (start 131.8164 103.124) (end 130.315 101.6226) (width 0.25) (layer "B.Cu") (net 18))
 (segment (start 131.484 96.432) (end 140.3719 96.432) (width 0.25) (layer "F.Cu") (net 16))
 (segment (start 130.556 95.504) (end 131.484 96.432) (width 0.25) (layer "F.Cu") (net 16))
 (segment (start 140.3719 96.432) (end 141.35 95.4539) (width 0.25) (layer "F.Cu") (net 16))
 (segment (start 141.35 95.4539) (end 141.35 94.45) (width 0.25) (layer "F.Cu") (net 16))
 (via (at 130.556 95.504) (size 0.6) (drill 0.3) (layers "F.Cu" "B.Cu") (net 16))
 (segment (start 128.6 82) (end 128.6 85) (width 0.25) (layer "B.Cu") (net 16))
 (segment (start 127.9225 93.4257) (end 129.3849 91.9633) (width 0.25) (layer "B.Cu") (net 16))
 (segment (start 129.3849 91.9633) (end 129.3849 85.7849) (width 0.25) (layer "B.Cu") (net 16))
 (segment (start 127.9225 94.4953) (end 127.9225 93.4257) (width 0.25) (layer "B.Cu") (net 16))
 (segment (start 128.9312 95.504) (end 127.9225 94.4953) (width 0.25) (layer "B.Cu") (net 16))
 (segment (start 129.3849 85.7849) (end 128.6 85) (width 0.25) (layer "B.Cu") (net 16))
 (segment (start 130.556 95.504) (end 128.9312 95.504) (width 0.25) (layer "B.Cu") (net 16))
 (segment (start 128.65 93.78) (end 130.65 91.78) (width 0.25) (layer "B.Cu") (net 15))
 (segment (start 128.65 94) (end 128.65 93.78) (width 0.25) (layer "B.Cu") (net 15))
 (segment (start 141.35 81.99) (end 141.35 83.77) (width 0.2) (layer "F.Cu") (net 20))
 (segment (start 134.362 97.278) (end 134.362 99.273) (width 0.2) (layer "F.Cu") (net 5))
 (segment (start 135.362 99.802) (end 135.362 100.298) (width 0.2) (layer "F.Cu") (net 5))
 (segment (start 134.3825 99.2935) (end 134.8535 99.2935) (width 0.2) (layer "F.Cu") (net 5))
 (segment (start 129.877 96.857) (end 133.941 96.857) (width 0.2) (layer "F.Cu") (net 5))
 (segment (start 133.941 96.857) (end 134.362 97.278) (width 0.2) (layer "F.Cu") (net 5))
 (segment (start 134.362 99.273) (end 134.3825 99.2935) (width 0.2) (layer "F.Cu") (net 5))
 (segment (start 130.65 93.56) (end 129.54 94.67) (width 0.2) (layer "F.Cu") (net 5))
 (segment (start 129.54 96.52) (end 129.877 96.857) (width 0.2) (layer "F.Cu") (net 5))
 (segment (start 129.54 94.67) (end 129.54 96.52) (width 0.2) (layer "F.Cu") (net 5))
 (segment (start 134.8535 99.2935) (end 135.362 99.802) (width 0.2) (layer "F.Cu") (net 5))
 (segment (start 130.65 93.56) (end 130.65 93.886) (width 0.2) (layer "B.Cu") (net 5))
 (segment (start 128.534232 100.838) (end 125.7571 98.060868) (width 0.25) (layer "F.Cu") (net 1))
 (segment (start 125.7571 87.0586) (end 129.2487 83.567) (width 0.25) (layer "F.Cu") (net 1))
 (segment (start 125.7571 98.060868) (end 125.7571 87.0586) (width 0.25) (layer "F.Cu") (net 1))
 (segment (start 133.362 100.298) (end 132.822 100.838) (width 0.25) (layer "F.Cu") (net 1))
 (segment (start 132.822 100.838) (end 128.534232 100.838) (width 0.25) (layer "F.Cu") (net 1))
 (via (at 129.2487 83.567) (size 0.6) (drill 0.3) (layers "F.Cu" "B.Cu") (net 1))
 (segment (start 129.6983 84.0166) (end 129.6983 84.66) (width 0.25) (layer "B.Cu") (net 1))
 (segment (start 130.65 84.66) (end 129.6983 84.66) (width 0.25) (layer "B.Cu") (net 1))
 (segment (start 129.2487 83.567) (end 129.6983 84.0166) (width 0.25) (layer "B.Cu") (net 1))
 (segment (start 133.862 97.823) (end 133.862 98.298) (width 0.25) (layer "F.Cu") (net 2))
 (segment (start 127.504531 97.278531) (end 128.778 97.278531) (width 0.25) (layer "F.Cu") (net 2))
 (segment (start 128.781469 97.282) (end 133.321 97.282) (width 0.25) (layer "F.Cu") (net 2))
 (segment (start 126.9193 96.6933) (end 127.504531 97.278531) (width 0.25) (layer "F.Cu") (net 2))
 (segment (start 127.1326 86.5827) (end 127.1326 92.4675) (width 0.25) (layer "F.Cu") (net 2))
 (segment (start 130.65 82.88) (end 130.65 83.0653) (width 0.25) (layer "F.Cu") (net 2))
 (segment (start 127.1326 92.4675) (end 126.9193 92.6808) (width 0.25) (layer "F.Cu") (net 2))
 (segment (start 126.9193 92.6808) (end 126.9193 96.6933) (width 0.25) (layer "F.Cu") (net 2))
 (segment (start 130.65 83.0653) (end 127.1326 86.5827) (width 0.25) (layer "F.Cu") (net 2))
 (segment (start 128.778 97.278531) (end 128.781469 97.282) (width 0.25) (layer "F.Cu") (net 2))
 (segment (start 133.321 97.282) (end 133.862 97.823) (width 0.25) (layer "F.Cu") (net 2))
 (segment (start 127.5402 92.7356) (end 127.5402 96.2982) (width 0.25) (layer "F.Cu") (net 3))
 (segment (start 134.62 100.556) (end 134.362 100.298) (width 0.25) (layer "F.Cu") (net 3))
 (segment (start 134.62 101.854) (end 134.62 100.556) (width 0.25) (layer "F.Cu") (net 3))
 (segment (start 127.895531 96.653531) (end 128.016 96.653531) (width 0.25) (layer "F.Cu") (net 3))
 (segment (start 130.65 88.22) (end 127.5843 91.2857) (width 0.25) (layer "F.Cu") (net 3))
 (segment (start 127.762 96.52) (end 127.895531 96.653531) (width 0.25) (layer "F.Cu") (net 3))
 (segment (start 130.307517 102.499001) (end 130.307518 102.499) (width 0.25) (layer "F.Cu") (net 3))
 (segment (start 127.5402 96.2982) (end 127.762 96.52) (width 0.25) (layer "F.Cu") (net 3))
 (segment (start 130.307518 102.499) (end 132.08 102.499) (width 0.25) (layer "F.Cu") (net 3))
 (segment (start 127.5843 92.6915) (end 127.5402 92.7356) (width 0.25) (layer "F.Cu") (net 3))
 (segment (start 127.5843 91.2857) (end 127.5843 92.6915) (width 0.25) (layer "F.Cu") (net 3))
 (via (at 130.307517 102.499001) (size 0.6) (drill 0.3) (layers "F.Cu" "B.Cu") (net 3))
 (via (at 128.016 96.653531) (size 0.6) (drill 0.3) (layers "F.Cu" "B.Cu") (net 3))
 (via (at 132.08 102.499) (size 0.6) (drill 0.3) (layers "F.Cu" "B.Cu") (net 3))
 (via (at 134.62 101.854) (size 0.6) (drill 0.3) (layers "F.Cu" "B.Cu") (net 3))
 (segment (start 129.54 100.076) (end 127.901052 98.437052) (width 0.25) (layer "B.Cu") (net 3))
 (segment (start 129.54 101.731484) (end 129.54 100.076) (width 0.25) (layer "B.Cu") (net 3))
 (segment (start 134.62 101.854) (end 133.975 102.499) (width 0.25) (layer "B.Cu") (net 3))
 (segment (start 133.975 102.499) (end 132.08 102.499) (width 0.25) (layer "B.Cu") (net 3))
 (segment (start 127.901052 98.437052) (end 127.901052 96.768479) (width 0.25) (layer "B.Cu") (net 3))
 (segment (start 130.307517 102.499001) (end 129.54 101.731484) (width 0.25) (layer "B.Cu") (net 3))
 (segment (start 127.901052 96.768479) (end 128.016 96.653531) (width 0.25) (layer "B.Cu") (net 3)))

